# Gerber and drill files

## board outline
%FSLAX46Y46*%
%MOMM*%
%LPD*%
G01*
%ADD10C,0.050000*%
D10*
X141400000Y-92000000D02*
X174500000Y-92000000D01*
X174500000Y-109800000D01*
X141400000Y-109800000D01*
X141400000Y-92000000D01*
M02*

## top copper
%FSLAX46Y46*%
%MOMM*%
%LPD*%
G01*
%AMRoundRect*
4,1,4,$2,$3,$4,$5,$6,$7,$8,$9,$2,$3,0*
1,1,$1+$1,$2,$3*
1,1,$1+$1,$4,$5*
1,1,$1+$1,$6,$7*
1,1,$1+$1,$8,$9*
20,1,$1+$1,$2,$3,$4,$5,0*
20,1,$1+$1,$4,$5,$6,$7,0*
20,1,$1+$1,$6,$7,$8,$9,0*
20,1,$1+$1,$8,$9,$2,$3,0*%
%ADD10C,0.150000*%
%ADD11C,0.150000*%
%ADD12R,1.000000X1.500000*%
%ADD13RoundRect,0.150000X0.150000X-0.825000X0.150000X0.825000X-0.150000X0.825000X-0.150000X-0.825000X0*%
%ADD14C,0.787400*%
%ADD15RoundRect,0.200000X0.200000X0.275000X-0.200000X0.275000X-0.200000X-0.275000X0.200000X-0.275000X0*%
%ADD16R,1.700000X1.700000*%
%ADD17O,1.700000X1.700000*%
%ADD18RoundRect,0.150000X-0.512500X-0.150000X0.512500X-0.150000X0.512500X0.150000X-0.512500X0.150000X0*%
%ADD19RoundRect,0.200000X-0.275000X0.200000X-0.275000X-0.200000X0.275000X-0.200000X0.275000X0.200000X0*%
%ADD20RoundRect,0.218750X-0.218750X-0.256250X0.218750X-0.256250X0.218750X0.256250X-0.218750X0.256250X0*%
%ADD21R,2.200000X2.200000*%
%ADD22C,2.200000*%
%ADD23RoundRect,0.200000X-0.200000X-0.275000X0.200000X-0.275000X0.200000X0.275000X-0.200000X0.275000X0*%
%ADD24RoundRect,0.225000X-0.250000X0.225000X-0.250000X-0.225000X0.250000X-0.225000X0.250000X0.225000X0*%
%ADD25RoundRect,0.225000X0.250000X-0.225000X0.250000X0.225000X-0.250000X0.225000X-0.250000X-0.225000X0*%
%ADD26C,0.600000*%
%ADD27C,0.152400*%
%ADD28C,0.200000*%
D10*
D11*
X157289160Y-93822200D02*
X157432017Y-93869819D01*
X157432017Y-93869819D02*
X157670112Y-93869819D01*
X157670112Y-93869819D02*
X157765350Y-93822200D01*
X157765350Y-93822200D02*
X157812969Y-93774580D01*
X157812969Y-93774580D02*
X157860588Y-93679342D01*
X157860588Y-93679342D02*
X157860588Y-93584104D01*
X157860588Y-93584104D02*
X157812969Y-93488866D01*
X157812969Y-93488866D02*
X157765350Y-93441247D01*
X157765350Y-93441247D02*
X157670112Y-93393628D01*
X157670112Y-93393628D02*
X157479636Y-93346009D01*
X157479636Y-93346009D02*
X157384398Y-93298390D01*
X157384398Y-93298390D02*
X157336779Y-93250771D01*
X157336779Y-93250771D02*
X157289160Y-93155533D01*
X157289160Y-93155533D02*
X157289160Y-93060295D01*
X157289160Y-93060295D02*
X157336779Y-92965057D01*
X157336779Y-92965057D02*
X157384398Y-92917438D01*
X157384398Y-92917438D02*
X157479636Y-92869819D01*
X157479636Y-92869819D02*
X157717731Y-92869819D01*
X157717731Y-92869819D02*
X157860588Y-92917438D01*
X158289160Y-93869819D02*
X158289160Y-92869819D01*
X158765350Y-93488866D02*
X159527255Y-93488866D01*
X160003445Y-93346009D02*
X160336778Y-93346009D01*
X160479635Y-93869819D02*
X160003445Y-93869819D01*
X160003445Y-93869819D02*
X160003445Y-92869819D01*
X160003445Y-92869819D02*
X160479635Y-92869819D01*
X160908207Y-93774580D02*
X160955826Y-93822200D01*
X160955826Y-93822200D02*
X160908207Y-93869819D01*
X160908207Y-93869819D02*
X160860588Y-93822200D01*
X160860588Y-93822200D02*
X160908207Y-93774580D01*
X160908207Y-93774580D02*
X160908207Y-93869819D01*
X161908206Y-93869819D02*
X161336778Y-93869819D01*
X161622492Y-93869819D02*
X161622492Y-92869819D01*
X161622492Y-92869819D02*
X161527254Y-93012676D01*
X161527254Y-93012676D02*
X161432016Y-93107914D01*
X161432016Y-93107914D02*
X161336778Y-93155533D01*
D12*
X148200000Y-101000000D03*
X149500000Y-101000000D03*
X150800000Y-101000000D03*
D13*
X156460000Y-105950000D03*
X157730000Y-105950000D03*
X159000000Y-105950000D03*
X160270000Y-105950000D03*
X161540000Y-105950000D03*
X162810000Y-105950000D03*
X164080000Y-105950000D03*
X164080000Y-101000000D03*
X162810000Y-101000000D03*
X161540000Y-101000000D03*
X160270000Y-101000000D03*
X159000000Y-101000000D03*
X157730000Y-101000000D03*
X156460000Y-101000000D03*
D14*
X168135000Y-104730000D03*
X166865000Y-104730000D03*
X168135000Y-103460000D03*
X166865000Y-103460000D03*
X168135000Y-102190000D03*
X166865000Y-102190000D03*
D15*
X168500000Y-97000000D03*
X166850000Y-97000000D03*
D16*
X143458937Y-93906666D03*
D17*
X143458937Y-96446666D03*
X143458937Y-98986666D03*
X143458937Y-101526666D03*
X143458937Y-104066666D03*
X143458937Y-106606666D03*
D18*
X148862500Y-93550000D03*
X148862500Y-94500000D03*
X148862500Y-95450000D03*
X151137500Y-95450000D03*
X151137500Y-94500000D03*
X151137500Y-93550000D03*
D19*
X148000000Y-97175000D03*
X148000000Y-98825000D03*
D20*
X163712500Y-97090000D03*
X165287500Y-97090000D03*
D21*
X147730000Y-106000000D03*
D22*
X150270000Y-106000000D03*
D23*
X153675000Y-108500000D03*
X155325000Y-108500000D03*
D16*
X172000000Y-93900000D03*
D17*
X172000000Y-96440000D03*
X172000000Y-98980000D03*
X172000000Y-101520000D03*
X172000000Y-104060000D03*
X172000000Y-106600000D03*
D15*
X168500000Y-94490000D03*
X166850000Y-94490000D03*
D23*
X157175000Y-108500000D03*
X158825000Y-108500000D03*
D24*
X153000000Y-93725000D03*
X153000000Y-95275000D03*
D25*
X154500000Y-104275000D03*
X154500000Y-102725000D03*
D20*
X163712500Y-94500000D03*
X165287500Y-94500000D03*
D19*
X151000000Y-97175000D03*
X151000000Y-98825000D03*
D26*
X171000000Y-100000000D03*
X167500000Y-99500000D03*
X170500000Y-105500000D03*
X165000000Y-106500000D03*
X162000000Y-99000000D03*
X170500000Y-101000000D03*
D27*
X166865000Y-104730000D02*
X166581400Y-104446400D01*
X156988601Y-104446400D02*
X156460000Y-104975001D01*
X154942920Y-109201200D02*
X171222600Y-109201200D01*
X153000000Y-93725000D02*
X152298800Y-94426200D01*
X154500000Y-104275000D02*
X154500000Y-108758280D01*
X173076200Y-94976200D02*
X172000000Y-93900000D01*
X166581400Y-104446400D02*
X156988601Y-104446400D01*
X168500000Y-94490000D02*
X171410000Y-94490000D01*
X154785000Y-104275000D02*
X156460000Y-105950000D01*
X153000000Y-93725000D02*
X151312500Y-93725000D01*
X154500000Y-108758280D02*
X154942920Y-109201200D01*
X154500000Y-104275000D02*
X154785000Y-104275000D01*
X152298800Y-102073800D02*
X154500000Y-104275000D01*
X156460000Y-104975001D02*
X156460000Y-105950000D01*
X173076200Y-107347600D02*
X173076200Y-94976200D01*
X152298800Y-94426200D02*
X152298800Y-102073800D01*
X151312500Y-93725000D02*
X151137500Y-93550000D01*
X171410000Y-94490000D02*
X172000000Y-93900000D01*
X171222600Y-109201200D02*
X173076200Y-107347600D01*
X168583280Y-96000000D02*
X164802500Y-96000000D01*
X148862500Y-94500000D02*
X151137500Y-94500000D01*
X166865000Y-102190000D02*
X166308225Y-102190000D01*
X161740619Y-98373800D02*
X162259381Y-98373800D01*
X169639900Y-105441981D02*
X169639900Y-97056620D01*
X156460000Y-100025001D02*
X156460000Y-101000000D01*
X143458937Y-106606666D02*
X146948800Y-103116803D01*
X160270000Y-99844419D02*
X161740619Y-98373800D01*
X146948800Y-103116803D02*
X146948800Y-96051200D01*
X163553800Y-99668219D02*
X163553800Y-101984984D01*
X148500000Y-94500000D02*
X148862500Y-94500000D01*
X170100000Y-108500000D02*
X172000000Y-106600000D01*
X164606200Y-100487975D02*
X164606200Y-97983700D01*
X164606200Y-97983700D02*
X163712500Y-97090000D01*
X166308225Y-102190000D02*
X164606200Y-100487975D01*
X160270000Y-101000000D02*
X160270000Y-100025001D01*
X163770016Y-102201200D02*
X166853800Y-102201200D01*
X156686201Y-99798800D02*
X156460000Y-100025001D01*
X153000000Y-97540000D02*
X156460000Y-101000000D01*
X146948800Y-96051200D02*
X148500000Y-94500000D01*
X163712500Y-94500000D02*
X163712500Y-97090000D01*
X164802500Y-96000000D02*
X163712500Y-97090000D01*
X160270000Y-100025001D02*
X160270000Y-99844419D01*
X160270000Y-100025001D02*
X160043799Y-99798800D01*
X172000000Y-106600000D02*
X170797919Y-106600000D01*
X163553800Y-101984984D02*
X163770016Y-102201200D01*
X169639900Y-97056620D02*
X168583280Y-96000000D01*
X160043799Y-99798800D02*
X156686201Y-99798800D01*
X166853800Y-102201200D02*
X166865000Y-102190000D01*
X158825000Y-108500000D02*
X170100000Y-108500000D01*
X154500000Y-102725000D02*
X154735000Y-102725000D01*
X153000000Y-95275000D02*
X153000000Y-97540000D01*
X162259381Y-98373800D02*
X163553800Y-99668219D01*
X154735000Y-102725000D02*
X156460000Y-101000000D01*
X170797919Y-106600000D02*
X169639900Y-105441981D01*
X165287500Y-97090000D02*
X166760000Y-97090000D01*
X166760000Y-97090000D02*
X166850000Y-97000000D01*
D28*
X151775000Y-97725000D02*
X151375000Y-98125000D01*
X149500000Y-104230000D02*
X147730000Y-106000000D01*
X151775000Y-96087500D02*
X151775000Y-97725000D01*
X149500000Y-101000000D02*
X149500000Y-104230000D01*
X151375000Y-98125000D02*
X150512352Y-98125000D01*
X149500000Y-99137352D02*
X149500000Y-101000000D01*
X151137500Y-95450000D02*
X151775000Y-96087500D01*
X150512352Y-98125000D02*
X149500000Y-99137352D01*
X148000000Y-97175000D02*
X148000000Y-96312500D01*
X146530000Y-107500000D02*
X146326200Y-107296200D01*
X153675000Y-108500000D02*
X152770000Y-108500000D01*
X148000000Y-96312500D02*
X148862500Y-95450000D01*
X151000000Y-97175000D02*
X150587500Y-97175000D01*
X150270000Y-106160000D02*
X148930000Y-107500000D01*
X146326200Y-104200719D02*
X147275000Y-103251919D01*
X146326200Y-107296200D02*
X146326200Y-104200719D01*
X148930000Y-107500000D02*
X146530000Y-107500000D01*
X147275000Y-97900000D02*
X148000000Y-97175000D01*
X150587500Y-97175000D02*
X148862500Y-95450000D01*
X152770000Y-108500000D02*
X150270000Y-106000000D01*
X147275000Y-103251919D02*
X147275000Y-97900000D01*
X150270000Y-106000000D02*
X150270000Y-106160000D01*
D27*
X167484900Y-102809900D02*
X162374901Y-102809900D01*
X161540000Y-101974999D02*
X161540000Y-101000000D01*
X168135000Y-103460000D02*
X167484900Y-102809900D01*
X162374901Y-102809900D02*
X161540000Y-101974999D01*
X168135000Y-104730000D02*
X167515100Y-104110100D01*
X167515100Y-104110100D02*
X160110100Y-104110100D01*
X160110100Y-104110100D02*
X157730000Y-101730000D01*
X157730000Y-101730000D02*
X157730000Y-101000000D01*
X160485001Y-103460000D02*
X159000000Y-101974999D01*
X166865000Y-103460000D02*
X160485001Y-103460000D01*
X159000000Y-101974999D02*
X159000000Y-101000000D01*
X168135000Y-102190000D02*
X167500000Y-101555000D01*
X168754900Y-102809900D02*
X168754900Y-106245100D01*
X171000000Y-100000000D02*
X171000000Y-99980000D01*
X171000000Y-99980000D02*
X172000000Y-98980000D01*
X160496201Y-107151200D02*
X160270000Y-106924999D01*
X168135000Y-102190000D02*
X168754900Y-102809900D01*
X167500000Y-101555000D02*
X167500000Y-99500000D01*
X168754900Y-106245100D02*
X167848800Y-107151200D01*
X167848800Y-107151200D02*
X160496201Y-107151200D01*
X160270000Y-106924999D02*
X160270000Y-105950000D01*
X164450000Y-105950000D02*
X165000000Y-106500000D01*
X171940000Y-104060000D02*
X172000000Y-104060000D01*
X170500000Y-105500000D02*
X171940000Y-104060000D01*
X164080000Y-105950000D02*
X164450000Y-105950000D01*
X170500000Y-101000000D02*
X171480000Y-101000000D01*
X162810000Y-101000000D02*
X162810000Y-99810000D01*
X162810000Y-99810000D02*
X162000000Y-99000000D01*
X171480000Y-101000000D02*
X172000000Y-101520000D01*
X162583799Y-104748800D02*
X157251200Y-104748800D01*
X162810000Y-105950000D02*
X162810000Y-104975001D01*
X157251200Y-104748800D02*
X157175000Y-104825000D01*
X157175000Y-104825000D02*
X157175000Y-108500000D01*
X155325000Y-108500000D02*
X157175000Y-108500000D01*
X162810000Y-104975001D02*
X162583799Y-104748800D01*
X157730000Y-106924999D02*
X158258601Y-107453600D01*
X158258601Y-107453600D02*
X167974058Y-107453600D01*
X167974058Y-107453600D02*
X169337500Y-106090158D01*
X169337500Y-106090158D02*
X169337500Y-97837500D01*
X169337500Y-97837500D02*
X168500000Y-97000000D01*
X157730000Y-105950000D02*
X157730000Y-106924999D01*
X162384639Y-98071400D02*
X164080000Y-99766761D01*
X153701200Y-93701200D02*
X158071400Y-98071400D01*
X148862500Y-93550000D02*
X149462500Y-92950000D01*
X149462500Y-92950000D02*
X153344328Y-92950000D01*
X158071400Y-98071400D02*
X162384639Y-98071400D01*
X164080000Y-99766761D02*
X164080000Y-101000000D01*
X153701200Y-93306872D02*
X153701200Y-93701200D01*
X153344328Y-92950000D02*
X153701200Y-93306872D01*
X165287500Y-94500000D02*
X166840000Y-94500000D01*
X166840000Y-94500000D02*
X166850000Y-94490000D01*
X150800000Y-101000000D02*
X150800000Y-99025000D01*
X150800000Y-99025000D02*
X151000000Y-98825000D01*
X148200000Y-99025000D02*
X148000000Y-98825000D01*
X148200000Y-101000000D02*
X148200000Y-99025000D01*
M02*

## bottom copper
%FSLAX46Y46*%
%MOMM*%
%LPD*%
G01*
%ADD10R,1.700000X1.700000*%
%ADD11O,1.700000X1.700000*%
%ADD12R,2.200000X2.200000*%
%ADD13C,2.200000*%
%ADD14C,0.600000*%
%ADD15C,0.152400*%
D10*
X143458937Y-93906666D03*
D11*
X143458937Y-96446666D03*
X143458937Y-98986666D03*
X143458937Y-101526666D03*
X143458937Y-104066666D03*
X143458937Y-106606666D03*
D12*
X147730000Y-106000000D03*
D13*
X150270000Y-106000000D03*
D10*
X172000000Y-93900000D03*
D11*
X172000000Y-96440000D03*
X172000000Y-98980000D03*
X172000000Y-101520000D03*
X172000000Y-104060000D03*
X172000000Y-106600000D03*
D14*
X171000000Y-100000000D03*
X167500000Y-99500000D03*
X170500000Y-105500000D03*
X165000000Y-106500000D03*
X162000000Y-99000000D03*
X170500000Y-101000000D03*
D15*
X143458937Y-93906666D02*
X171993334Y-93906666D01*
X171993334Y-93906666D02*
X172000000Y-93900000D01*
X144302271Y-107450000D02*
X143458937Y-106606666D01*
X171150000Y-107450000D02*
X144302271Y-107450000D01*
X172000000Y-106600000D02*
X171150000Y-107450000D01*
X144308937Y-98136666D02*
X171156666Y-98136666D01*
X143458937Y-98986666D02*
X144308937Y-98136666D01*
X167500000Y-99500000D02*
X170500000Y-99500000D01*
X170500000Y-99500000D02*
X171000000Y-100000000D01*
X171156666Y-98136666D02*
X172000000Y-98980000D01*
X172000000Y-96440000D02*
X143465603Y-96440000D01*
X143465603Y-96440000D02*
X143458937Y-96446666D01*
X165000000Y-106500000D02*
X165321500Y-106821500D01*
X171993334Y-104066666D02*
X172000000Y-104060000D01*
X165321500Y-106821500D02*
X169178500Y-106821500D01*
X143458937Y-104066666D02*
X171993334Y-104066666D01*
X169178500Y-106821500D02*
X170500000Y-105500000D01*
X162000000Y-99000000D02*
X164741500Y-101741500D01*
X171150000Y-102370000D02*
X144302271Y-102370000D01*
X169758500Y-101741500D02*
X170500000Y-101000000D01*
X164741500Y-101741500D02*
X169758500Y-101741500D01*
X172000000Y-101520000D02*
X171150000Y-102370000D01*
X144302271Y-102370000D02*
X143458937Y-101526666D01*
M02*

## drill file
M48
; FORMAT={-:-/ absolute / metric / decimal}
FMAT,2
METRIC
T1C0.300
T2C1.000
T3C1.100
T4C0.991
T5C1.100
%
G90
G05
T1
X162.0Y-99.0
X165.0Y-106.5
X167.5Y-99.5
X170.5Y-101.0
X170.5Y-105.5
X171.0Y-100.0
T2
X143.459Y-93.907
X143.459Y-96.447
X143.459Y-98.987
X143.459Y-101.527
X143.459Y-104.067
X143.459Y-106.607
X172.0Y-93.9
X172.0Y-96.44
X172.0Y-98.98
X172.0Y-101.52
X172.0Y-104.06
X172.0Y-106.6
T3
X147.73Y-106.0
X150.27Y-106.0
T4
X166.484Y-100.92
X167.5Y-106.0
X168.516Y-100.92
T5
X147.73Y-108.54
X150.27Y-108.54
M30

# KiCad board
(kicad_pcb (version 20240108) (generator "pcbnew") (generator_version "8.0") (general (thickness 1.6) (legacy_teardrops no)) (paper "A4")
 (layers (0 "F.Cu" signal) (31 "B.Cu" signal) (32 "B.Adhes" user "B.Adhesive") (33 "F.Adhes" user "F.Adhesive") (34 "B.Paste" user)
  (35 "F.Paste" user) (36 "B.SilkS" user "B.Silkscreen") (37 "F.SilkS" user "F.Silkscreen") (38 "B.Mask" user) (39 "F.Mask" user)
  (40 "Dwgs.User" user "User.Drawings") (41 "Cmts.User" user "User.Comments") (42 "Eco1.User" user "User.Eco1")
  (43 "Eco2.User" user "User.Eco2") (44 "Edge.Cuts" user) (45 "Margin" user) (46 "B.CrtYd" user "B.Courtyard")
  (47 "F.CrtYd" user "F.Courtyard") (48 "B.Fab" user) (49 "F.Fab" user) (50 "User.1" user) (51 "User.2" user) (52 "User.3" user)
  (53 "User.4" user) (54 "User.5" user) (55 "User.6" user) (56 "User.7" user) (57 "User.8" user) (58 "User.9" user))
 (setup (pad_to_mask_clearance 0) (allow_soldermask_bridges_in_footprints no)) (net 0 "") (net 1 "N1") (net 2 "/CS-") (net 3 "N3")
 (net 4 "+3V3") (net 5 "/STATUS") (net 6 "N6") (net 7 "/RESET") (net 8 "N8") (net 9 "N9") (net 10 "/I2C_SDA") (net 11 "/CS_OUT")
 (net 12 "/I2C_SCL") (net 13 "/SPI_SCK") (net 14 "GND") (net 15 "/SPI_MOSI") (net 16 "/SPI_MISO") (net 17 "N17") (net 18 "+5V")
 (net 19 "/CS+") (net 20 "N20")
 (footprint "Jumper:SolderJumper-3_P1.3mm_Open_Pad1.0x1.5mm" (layer "F.Cu") (at 149.5 101)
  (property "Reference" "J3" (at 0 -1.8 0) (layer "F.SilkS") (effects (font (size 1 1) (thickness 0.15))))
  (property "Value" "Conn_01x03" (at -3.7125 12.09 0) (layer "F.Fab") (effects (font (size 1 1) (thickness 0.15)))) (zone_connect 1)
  (pad "1" smd rect (at -1.3 0) (size 1 1.5) (layers "F.Cu" "F.Mask") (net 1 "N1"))
  (pad "2" smd rect (at 0 0) (size 1 1.5) (layers "F.Cu" "F.Mask") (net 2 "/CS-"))
  (pad "3" smd rect (at 1.3 0) (size 1 1.5) (layers "F.Cu" "F.Mask") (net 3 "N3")))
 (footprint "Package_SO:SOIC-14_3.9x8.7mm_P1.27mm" (layer "F.Cu") (at 160.27 103.475 90)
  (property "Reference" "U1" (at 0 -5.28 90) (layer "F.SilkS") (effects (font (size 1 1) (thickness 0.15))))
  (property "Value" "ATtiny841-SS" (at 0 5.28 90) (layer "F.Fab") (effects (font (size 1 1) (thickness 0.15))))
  (pad "1" smd roundrect (at -2.475 -3.81 90) (size 1.95 0.6) (layers "F.Cu" "F.Paste" "F.Mask") (roundrect_rratio 0.25) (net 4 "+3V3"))
  (pad "2" smd roundrect (at -2.475 -2.54 90) (size 1.95 0.6) (layers "F.Cu" "F.Paste" "F.Mask") (roundrect_rratio 0.25) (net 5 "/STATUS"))
  (pad "3" smd roundrect (at -2.475 -1.27 90) (size 1.95 0.6) (layers "F.Cu" "F.Paste" "F.Mask") (roundrect_rratio 0.25) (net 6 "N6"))
  (pad "4" smd roundrect (at -2.475 0 90) (size 1.95 0.6) (layers "F.Cu" "F.Paste" "F.Mask") (roundrect_rratio 0.25) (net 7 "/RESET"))
  (pad "5" smd roundrect (at -2.475 1.27 90) (size 1.95 0.6) (layers "F.Cu" "F.Paste" "F.Mask") (roundrect_rratio 0.25) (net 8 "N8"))
  (pad "6" smd roundrect (at -2.475 2.54 90) (size 1.95 0.6) (layers "F.Cu" "F.Paste" "F.Mask") (roundrect_rratio 0.25) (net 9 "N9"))
  (pad "7" smd roundrect (at -2.475 3.81 90) (size 1.95 0.6) (layers "F.Cu" "F.Paste" "F.Mask") (roundrect_rratio 0.25) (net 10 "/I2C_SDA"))
  (pad "8" smd roundrect (at 2.475 3.81 90) (size 1.95 0.6) (layers "F.Cu" "F.Paste" "F.Mask") (roundrect_rratio 0.25) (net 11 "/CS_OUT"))
  (pad "9" smd roundrect (at 2.475 2.54 90) (size 1.95 0.6) (layers "F.Cu" "F.Paste" "F.Mask") (roundrect_rratio 0.25) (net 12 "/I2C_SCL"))
  (pad "10" smd roundrect (at 2.475 1.27 90) (size 1.95 0.6) (layers "F.Cu" "F.Paste" "F.Mask") (roundrect_rratio 0.25) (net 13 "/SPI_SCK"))
  (pad "11" smd roundrect (at 2.475 0 90) (size 1.95 0.6) (layers "F.Cu" "F.Paste" "F.Mask") (roundrect_rratio 0.25) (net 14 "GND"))
  (pad "12" smd roundrect (at 2.475 -1.27 90) (size 1.95 0.6) (layers "F.Cu" "F.Paste" "F.Mask") (roundrect_rratio 0.25)
   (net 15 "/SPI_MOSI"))
  (pad "13" smd roundrect (at 2.475 -2.54 90) (size 1.95 0.6) (layers "F.Cu" "F.Paste" "F.Mask") (roundrect_rratio 0.25)
   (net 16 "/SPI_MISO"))
  (pad "14" smd roundrect (at 2.475 -3.81 90) (size 1.95 0.6) (layers "F.Cu" "F.Paste" "F.Mask") (roundrect_rratio 0.25) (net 14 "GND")))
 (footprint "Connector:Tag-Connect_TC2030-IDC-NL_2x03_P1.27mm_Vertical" (layer "F.Cu") (at 167.5 103.46 90)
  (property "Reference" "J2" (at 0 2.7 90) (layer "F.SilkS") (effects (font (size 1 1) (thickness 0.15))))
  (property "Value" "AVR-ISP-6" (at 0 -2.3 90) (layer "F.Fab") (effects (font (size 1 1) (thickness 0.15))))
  (pad "" np_thru_hole circle (at -2.54 0 90) (size 0.9906 0.9906) (drill 0.9906) (layers "*.Cu" "*.Mask"))
  (pad "" np_thru_hole circle (at 2.54 -1.016 90) (size 0.9906 0.9906) (drill 0.9906) (layers "*.Cu" "*.Mask"))
  (pad "" np_thru_hole circle (at 2.54 1.016 90) (size 0.9906 0.9906) (drill 0.9906) (layers "*.Cu" "*.Mask"))
  (pad "1" connect circle (at -1.27 0.635 90) (size 0.7874 0.7874) (layers "F.Cu" "F.Mask") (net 16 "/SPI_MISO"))
  (pad "2" connect circle (at -1.27 -0.635 90) (size 0.7874 0.7874) (layers "F.Cu" "F.Mask") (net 4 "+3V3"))
  (pad "3" connect circle (at 0 0.635 90) (size 0.7874 0.7874) (layers "F.Cu" "F.Mask") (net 13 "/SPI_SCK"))
  (pad "4" connect circle (at 0 -0.635 90) (size 0.7874 0.7874) (layers "F.Cu" "F.Mask") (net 15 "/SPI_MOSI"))
  (pad "5" connect circle (at 1.27 0.635 90) (size 0.7874 0.7874) (layers "F.Cu" "F.Mask") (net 7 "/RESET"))
  (pad "6" connect circle (at 1.27 -0.635 90) (size 0.7874 0.7874) (layers "F.Cu" "F.Mask") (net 14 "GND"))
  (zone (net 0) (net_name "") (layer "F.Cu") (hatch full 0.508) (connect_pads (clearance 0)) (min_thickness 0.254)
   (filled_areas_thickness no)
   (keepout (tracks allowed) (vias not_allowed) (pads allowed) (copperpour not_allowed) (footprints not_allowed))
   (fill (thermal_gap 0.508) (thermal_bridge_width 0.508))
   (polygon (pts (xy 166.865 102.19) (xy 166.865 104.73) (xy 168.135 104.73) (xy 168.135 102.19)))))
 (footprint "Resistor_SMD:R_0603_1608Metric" (layer "F.Cu") (at 167.675 97 180)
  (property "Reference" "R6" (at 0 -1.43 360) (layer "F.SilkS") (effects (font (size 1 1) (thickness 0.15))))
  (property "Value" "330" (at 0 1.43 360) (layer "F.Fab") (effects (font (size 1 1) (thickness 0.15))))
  (pad "1" smd roundrect (at -0.825 0 180) (size 0.8 0.95) (layers "F.Cu" "F.Paste" "F.Mask") (roundrect_rratio 0.25) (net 5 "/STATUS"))
  (pad "2" smd roundrect (at 0.825 0 180) (size 0.8 0.95) (layers "F.Cu" "F.Paste" "F.Mask") (roundrect_rratio 0.25) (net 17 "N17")))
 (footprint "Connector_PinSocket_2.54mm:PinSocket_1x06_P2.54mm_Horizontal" (layer "F.Cu") (at 143.458937 93.906666)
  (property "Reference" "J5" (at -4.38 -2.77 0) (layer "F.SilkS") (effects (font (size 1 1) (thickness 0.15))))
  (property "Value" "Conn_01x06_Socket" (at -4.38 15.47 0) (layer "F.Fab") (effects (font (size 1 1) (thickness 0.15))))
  (pad "1" thru_hole rect (at 0 0) (size 1.7 1.7) (drill 1) (layers "*.Cu" "*.Mask") (remove_unused_layers no) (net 4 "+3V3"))
  (pad "2" thru_hole oval (at 0 2.54) (size 1.7 1.7) (drill 1) (layers "*.Cu" "*.Mask") (remove_unused_layers no) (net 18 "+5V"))
  (pad "3" thru_hole oval (at 0 5.08) (size 1.7 1.7) (drill 1) (layers "*.Cu" "*.Mask") (remove_unused_layers no) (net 7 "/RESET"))
  (pad "4" thru_hole oval (at 0 7.62) (size 1.7 1.7) (drill 1) (layers "*.Cu" "*.Mask") (remove_unused_layers no) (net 12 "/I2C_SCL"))
  (pad "5" thru_hole oval (at 0 10.16) (size 1.7 1.7) (drill 1) (layers "*.Cu" "*.Mask") (remove_unused_layers no) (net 10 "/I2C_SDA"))
  (pad "6" thru_hole oval (at 0 12.7) (size 1.7 1.7) (drill 1) (layers "*.Cu" "*.Mask") (remove_unused_layers no) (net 14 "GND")))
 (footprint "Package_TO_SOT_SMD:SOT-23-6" (layer "F.Cu") (at 150 94.5)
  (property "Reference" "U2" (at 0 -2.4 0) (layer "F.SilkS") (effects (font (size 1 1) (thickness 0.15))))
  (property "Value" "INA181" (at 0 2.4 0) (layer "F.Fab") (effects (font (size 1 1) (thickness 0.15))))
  (pad "1" smd roundrect (at -1.1375 -0.95) (size 1.325 0.6) (layers "F.Cu" "F.Paste" "F.Mask") (roundrect_rratio 0.25) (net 11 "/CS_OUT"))
  (pad "2" smd roundrect (at -1.1375 0) (size 1.325 0.6) (layers "F.Cu" "F.Paste" "F.Mask") (roundrect_rratio 0.25) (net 14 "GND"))
  (pad "3" smd roundrect (at -1.1375 0.95) (size 1.325 0.6) (layers "F.Cu" "F.Paste" "F.Mask") (roundrect_rratio 0.25) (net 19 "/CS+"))
  (pad "4" smd roundrect (at 1.1375 0.95) (size 1.325 0.6) (layers "F.Cu" "F.Paste" "F.Mask") (roundrect_rratio 0.25) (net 2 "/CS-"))
  (pad "5" smd roundrect (at 1.1375 0) (size 1.325 0.6) (layers "F.Cu" "F.Paste" "F.Mask") (roundrect_rratio 0.25) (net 14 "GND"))
  (pad "6" smd roundrect (at 1.1375 -0.95) (size 1.325 0.6) (layers "F.Cu" "F.Paste" "F.Mask") (roundrect_rratio 0.25) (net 4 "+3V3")))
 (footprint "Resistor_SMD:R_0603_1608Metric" (layer "F.Cu") (at 148 98 -90)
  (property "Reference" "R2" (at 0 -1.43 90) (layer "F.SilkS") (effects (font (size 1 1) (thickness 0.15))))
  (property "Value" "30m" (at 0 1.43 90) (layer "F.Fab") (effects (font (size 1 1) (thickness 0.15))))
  (pad "1" smd roundrect (at -0.825 0 270) (size 0.8 0.95) (layers "F.Cu" "F.Paste" "F.Mask") (roundrect_rratio 0.25) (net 19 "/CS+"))
  (pad "2" smd roundrect (at 0.825 0 270) (size 0.8 0.95) (layers "F.Cu" "F.Paste" "F.Mask") (roundrect_rratio 0.25) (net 1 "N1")))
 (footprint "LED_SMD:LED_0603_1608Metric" (layer "F.Cu") (at 164.5 97.09)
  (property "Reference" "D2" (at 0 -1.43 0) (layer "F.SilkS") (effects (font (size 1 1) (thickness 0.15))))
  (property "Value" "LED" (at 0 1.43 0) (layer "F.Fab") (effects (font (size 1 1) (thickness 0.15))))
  (pad "1" smd roundrect (at -0.7875 0) (size 0.875 0.95) (layers "F.Cu" "F.Paste" "F.Mask") (roundrect_rratio 0.25) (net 14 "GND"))
  (pad "2" smd roundrect (at 0.7875 0) (size 0.875 0.95) (layers "F.Cu" "F.Paste" "F.Mask") (roundrect_rratio 0.25) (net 17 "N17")))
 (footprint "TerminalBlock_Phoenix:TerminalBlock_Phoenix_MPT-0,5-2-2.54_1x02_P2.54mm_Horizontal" (layer "F.Cu") (at 147.73 106)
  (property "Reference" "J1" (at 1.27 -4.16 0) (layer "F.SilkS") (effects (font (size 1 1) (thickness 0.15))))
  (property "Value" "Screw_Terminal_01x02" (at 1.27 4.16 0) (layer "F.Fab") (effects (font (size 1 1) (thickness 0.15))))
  (pad "" np_thru_hole circle (at 0 2.54) (size 1.1 1.1) (drill 1.1) (layers "*.Cu" "*.Mask"))
  (pad "" np_thru_hole circle (at 2.54 2.54) (size 1.1 1.1) (drill 1.1) (layers "*.Cu" "*.Mask"))
  (pad "1" thru_hole rect (at 0 0) (size 2.2 2.2) (drill 1.1) (layers "*.Cu" "*.Mask") (remove_unused_layers no) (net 2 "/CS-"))
  (pad "2" thru_hole circle (at 2.54 0) (size 2.2 2.2) (drill 1.1) (layers "*.Cu" "*.Mask") (remove_unused_layers no) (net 19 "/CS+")))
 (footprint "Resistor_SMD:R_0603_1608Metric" (layer "F.Cu") (at 154.5 108.5)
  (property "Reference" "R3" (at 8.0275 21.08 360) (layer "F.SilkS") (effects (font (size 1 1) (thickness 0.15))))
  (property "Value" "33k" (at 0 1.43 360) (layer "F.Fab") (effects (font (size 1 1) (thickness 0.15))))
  (pad "1" smd roundrect (at -0.825 0) (size 0.8 0.95) (layers "F.Cu" "F.Paste" "F.Mask") (roundrect_rratio 0.25) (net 19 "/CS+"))
  (pad "2" smd roundrect (at 0.825 0) (size 0.8 0.95) (layers "F.Cu" "F.Paste" "F.Mask") (roundrect_rratio 0.25) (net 9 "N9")))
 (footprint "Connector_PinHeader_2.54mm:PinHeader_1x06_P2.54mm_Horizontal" (layer "F.Cu") (at 172 93.9)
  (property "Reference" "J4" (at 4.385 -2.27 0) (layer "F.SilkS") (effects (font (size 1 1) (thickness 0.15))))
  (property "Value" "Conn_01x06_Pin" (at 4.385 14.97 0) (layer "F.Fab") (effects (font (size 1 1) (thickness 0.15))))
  (pad "1" thru_hole rect (at 0 0) (size 1.7 1.7) (drill 1) (layers "*.Cu" "*.Mask") (remove_unused_layers no) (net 4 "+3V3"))
  (pad "2" thru_hole oval (at 0 2.54) (size 1.7 1.7) (drill 1) (layers "*.Cu" "*.Mask") (remove_unused_layers no) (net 18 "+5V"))
  (pad "3" thru_hole oval (at 0 5.08) (size 1.7 1.7) (drill 1) (layers "*.Cu" "*.Mask") (remove_unused_layers no) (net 7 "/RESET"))
  (pad "4" thru_hole oval (at 0 7.62) (size 1.7 1.7) (drill 1) (layers "*.Cu" "*.Mask") (remove_unused_layers no) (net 12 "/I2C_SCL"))
  (pad "5" thru_hole oval (at 0 10.16) (size 1.7 1.7) (drill 1) (layers "*.Cu" "*.Mask") (remove_unused_layers no) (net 10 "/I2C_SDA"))
  (pad "6" thru_hole oval (at 0 12.7) (size 1.7 1.7) (drill 1) (layers "*.Cu" "*.Mask") (remove_unused_layers no) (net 14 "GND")))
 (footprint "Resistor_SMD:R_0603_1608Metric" (layer "F.Cu") (at 167.675 94.49 180)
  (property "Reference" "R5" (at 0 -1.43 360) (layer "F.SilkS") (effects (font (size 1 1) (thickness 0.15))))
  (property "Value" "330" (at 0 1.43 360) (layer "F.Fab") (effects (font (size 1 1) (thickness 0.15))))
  (pad "1" smd roundrect (at -0.825 0 180) (size 0.8 0.95) (layers "F.Cu" "F.Paste" "F.Mask") (roundrect_rratio 0.25) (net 4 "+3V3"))
  (pad "2" smd roundrect (at 0.825 0 180) (size 0.8 0.95) (layers "F.Cu" "F.Paste" "F.Mask") (roundrect_rratio 0.25) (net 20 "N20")))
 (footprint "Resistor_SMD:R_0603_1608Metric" (layer "F.Cu") (at 158 108.5)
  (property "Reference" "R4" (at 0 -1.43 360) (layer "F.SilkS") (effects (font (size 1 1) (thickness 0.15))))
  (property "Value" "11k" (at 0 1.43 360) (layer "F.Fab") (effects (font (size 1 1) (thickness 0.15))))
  (pad "1" smd roundrect (at -0.825 0) (size 0.8 0.95) (layers "F.Cu" "F.Paste" "F.Mask") (roundrect_rratio 0.25) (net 9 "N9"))
  (pad "2" smd roundrect (at 0.825 0) (size 0.8 0.95) (layers "F.Cu" "F.Paste" "F.Mask") (roundrect_rratio 0.25) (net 14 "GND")))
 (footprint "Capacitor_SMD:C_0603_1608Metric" (layer "F.Cu") (at 153 94.5 -90)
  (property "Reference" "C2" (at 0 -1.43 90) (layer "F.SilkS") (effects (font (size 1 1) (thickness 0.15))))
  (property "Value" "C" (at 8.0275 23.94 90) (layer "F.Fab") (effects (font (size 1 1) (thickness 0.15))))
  (pad "1" smd roundrect (at -0.775 0 270) (size 0.9 0.95) (layers "F.Cu" "F.Paste" "F.Mask") (roundrect_rratio 0.25) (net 4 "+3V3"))
  (pad "2" smd roundrect (at 0.775 0 270) (size 0.9 0.95) (layers "F.Cu" "F.Paste" "F.Mask") (roundrect_rratio 0.25) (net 14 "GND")))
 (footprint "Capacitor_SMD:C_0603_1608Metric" (layer "F.Cu") (at 154.5 103.5 90)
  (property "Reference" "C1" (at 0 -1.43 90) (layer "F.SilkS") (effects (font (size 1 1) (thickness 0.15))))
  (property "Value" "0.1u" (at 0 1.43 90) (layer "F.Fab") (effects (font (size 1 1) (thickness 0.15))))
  (pad "1" smd roundrect (at -0.775 0 90) (size 0.9 0.95) (layers "F.Cu" "F.Paste" "F.Mask") (roundrect_rratio 0.25) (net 4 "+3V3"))
  (pad "2" smd roundrect (at 0.775 0 90) (size 0.9 0.95) (layers "F.Cu" "F.Paste" "F.Mask") (roundrect_rratio 0.25) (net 14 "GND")))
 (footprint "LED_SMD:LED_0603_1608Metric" (layer "F.Cu") (at 164.5 94.5)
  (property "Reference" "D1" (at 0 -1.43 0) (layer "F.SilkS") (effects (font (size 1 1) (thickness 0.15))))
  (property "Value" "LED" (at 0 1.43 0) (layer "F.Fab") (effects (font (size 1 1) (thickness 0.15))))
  (pad "1" smd roundrect (at -0.7875 0) (size 0.875 0.95) (layers "F.Cu" "F.Paste" "F.Mask") (roundrect_rratio 0.25) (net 14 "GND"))
  (pad "2" smd roundrect (at 0.7875 0) (size 0.875 0.95) (layers "F.Cu" "F.Paste" "F.Mask") (roundrect_rratio 0.25) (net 20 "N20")))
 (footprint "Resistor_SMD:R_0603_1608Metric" (layer "F.Cu") (at 151 98 -90)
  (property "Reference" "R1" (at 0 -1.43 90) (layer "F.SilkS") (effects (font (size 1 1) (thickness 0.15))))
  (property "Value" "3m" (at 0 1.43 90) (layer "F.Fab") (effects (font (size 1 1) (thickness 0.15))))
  (pad "1" smd roundrect (at -0.825 0 270) (size 0.8 0.95) (layers "F.Cu" "F.Paste" "F.Mask") (roundrect_rratio 0.25) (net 19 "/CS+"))
  (pad "2" smd roundrect (at 0.825 0 270) (size 0.8 0.95) (layers "F.Cu" "F.Paste" "F.Mask") (roundrect_rratio 0.25) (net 3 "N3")))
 (gr_rect (start 141.4 92) (end 174.5 109.8) (stroke (width 0.05) (type default)) (fill none) (layer "Edge.Cuts"))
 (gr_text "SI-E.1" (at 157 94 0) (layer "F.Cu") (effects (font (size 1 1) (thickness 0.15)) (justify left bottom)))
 (segment (start 166.865 104.73) (end 166.5814 104.4464) (width 0.1524) (layer "F.Cu") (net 4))
 (segment (start 156.988601 104.4464) (end 156.46 104.975001) (width 0.1524) (layer "F.Cu") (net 4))
 (segment (start 154.94292 109.2012) (end 171.2226 109.2012) (width 0.1524) (layer "F.Cu") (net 4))
 (segment (start 153 93.725) (end 152.2988 94.4262) (width 0.1524) (layer "F.Cu") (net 4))
 (segment (start 154.5 104.275) (end 154.5 108.75828) (width 0.1524) (layer "F.Cu") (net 4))
 (segment (start 173.0762 94.9762) (end 172 93.9) (width 0.1524) (layer "F.Cu") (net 4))
 (segment (start 166.5814 104.4464) (end 156.988601 104.4464) (width 0.1524) (layer "F.Cu") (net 4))
 (segment (start 168.5 94.49) (end 171.41 94.49) (width 0.1524) (layer "F.Cu") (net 4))
 (segment (start 154.785 104.275) (end 156.46 105.95) (width 0.1524) (layer "F.Cu") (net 4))
 (segment (start 153 93.725) (end 151.3125 93.725) (width 0.1524) (layer "F.Cu") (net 4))
 (segment (start 154.5 108.75828) (end 154.94292 109.2012) (width 0.1524) (layer "F.Cu") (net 4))
 (segment (start 154.5 104.275) (end 154.785 104.275) (width 0.1524) (layer "F.Cu") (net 4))
 (segment (start 152.2988 102.0738) (end 154.5 104.275) (width 0.1524) (layer "F.Cu") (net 4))
 (segment (start 156.46 104.975001) (end 156.46 105.95) (width 0.1524) (layer "F.Cu") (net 4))
 (segment (start 173.0762 107.3476) (end 173.0762 94.9762) (width 0.1524) (layer "F.Cu") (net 4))
 (segment (start 152.2988 94.4262) (end 152.2988 102.0738) (width 0.1524) (layer "F.Cu") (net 4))
 (segment (start 151.3125 93.725) (end 151.1375 93.55) (width 0.1524) (layer "F.Cu") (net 4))
 (segment (start 171.41 94.49) (end 172 93.9) (width 0.1524) (layer "F.Cu") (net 4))
 (segment (start 171.2226 109.2012) (end 173.0762 107.3476) (width 0.1524) (layer "F.Cu") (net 4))
 (segment (start 143.458937 93.906666) (end 171.993334 93.906666) (width 0.1524) (layer "B.Cu") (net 4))
 (segment (start 171.993334 93.906666) (end 172 93.9) (width 0.1524) (layer "B.Cu") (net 4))
 (segment (start 168.58328 96) (end 164.8025 96) (width 0.1524) (layer "F.Cu") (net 14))
 (segment (start 148.8625 94.5) (end 151.1375 94.5) (width 0.1524) (layer "F.Cu") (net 14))
 (segment (start 166.865 102.19) (end 166.308225 102.19) (width 0.1524) (layer "F.Cu") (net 14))
 (segment (start 161.740619 98.3738) (end 162.259381 98.3738) (width 0.1524) (layer "F.Cu") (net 14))
 (segment (start 169.6399 105.441981) (end 169.6399 97.05662) (width 0.1524) (layer "F.Cu") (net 14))
 (segment (start 156.46 100.025001) (end 156.46 101) (width 0.1524) (layer "F.Cu") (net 14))
 (segment (start 143.458937 106.606666) (end 146.9488 103.116803) (width 0.1524) (layer "F.Cu") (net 14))
 (segment (start 160.27 99.844419) (end 161.740619 98.3738) (width 0.1524) (layer "F.Cu") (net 14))
 (segment (start 146.9488 103.116803) (end 146.9488 96.0512) (width 0.1524) (layer "F.Cu") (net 14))
 (segment (start 163.5538 99.668219) (end 163.5538 101.984984) (width 0.1524) (layer "F.Cu") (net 14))
 (segment (start 148.5 94.5) (end 148.8625 94.5) (width 0.1524) (layer "F.Cu") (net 14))
 (segment (start 170.1 108.5) (end 172 106.6) (width 0.1524) (layer "F.Cu") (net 14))
 (segment (start 164.6062 100.487975) (end 164.6062 97.9837) (width 0.1524) (layer "F.Cu") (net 14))
 (segment (start 164.6062 97.9837) (end 163.7125 97.09) (width 0.1524) (layer "F.Cu") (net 14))
 (segment (start 166.308225 102.19) (end 164.6062 100.487975) (width 0.1524) (layer "F.Cu") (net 14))
 (segment (start 160.27 101) (end 160.27 100.025001) (width 0.1524) (layer "F.Cu") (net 14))
 (segment (start 163.770016 102.2012) (end 166.8538 102.2012) (width 0.1524) (layer "F.Cu") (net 14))
 (segment (start 156.686201 99.7988) (end 156.46 100.025001) (width 0.1524) (layer "F.Cu") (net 14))
 (segment (start 153 97.54) (end 156.46 101) (width 0.1524) (layer "F.Cu") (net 14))
 (segment (start 146.9488 96.0512) (end 148.5 94.5) (width 0.1524) (layer "F.Cu") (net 14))
 (segment (start 163.7125 94.5) (end 163.7125 97.09) (width 0.1524) (layer "F.Cu") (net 14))
 (segment (start 164.8025 96) (end 163.7125 97.09) (width 0.1524) (layer "F.Cu") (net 14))
 (segment (start 160.27 100.025001) (end 160.27 99.844419) (width 0.1524) (layer "F.Cu") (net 14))
 (segment (start 160.27 100.025001) (end 160.043799 99.7988) (width 0.1524) (layer "F.Cu") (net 14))
 (segment (start 172 106.6) (end 170.797919 106.6) (width 0.1524) (layer "F.Cu") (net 14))
 (segment (start 163.5538 101.984984) (end 163.770016 102.2012) (width 0.1524) (layer "F.Cu") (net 14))
 (segment (start 169.6399 97.05662) (end 168.58328 96) (width 0.1524) (layer "F.Cu") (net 14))
 (segment (start 160.043799 99.7988) (end 156.686201 99.7988) (width 0.1524) (layer "F.Cu") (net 14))
 (segment (start 166.8538 102.2012) (end 166.865 102.19) (width 0.1524) (layer "F.Cu") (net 14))
 (segment (start 158.825 108.5) (end 170.1 108.5) (width 0.1524) (layer "F.Cu") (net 14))
 (segment (start 154.5 102.725) (end 154.735 102.725) (width 0.1524) (layer "F.Cu") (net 14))
 (segment (start 153 95.275) (end 153 97.54) (width 0.1524) (layer "F.Cu") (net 14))
 (segment (start 162.259381 98.3738) (end 163.5538 99.668219) (width 0.1524) (layer "F.Cu") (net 14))
 (segment (start 154.735 102.725) (end 156.46 101) (width 0.1524) (layer "F.Cu") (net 14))
 (segment (start 170.797919 106.6) (end 169.6399 105.441981) (width 0.1524) (layer "F.Cu") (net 14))
 (segment (start 144.302271 107.45) (end 143.458937 106.606666) (width 0.1524) (layer "B.Cu") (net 14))
 (segment (start 171.15 107.45) (end 144.302271 107.45) (width 0.1524) (layer "B.Cu") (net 14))
 (segment (start 172 106.6) (end 171.15 107.45) (width 0.1524) (layer "B.Cu") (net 14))
 (segment (start 165.2875 97.09) (end 166.76 97.09) (width 0.1524) (layer "F.Cu") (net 17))
 (segment (start 166.76 97.09) (end 166.85 97) (width 0.1524) (layer "F.Cu") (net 17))
 (segment (start 151.775 97.725) (end 151.375 98.125) (width 0.2) (layer "F.Cu") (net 2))
 (segment (start 149.5 104.23) (end 147.73 106) (width 0.2) (layer "F.Cu") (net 2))
 (segment (start 151.775 96.0875) (end 151.775 97.725) (width 0.2) (layer "F.Cu") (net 2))
 (segment (start 149.5 101) (end 149.5 104.23) (width 0.2) (layer "F.Cu") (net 2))
 (segment (start 151.375 98.125) (end 150.512352 98.125) (width 0.2) (layer "F.Cu") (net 2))
 (segment (start 149.5 99.137352) (end 149.5 101) (width 0.2) (layer "F.Cu") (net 2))
 (segment (start 151.1375 95.45) (end 151.775 96.0875) (width 0.2) (layer "F.Cu") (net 2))
 (segment (start 150.512352 98.125) (end 149.5 99.137352) (width 0.2) (layer "F.Cu") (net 2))
 (segment (start 148 97.175) (end 148 96.3125) (width 0.2) (layer "F.Cu") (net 19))
 (segment (start 146.53 107.5) (end 146.3262 107.2962) (width 0.2) (layer "F.Cu") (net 19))
 (segment (start 153.675 108.5) (end 152.77 108.5) (width 0.2) (layer "F.Cu") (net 19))
 (segment (start 148 96.3125) (end 148.8625 95.45) (width 0.2) (layer "F.Cu") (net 19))
 (segment (start 151 97.175) (end 150.5875 97.175) (width 0.2) (layer "F.Cu") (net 19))
 (segment (start 150.27 106.16) (end 148.93 107.5) (width 0.2) (layer "F.Cu") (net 19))
 (segment (start 146.3262 104.200719) (end 147.275 103.251919) (width 0.2) (layer "F.Cu") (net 19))
 (segment (start 146.3262 107.2962) (end 146.3262 104.200719) (width 0.2) (layer "F.Cu") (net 19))
 (segment (start 148.93 107.5) (end 146.53 107.5) (width 0.2) (layer "F.Cu") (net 19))
 (segment (start 147.275 97.9) (end 148 97.175) (width 0.2) (layer "F.Cu") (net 19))
 (segment (start 150.5875 97.175) (end 148.8625 95.45) (width 0.2) (layer "F.Cu") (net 19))
 (segment (start 152.77 108.5) (end 150.27 106) (width 0.2) (layer "F.Cu") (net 19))
 (segment (start 147.275 103.251919) (end 147.275 97.9) (width 0.2) (layer "F.Cu") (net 19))
 (segment (start 150.27 106) (end 150.27 106.16) (width 0.2) (layer "F.Cu") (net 19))
 (segment (start 167.4849 102.8099) (end 162.374901 102.8099) (width 0.1524) (layer "F.Cu") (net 13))
 (segment (start 161.54 101.974999) (end 161.54 101) (width 0.1524) (layer "F.Cu") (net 13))
 (segment (start 168.135 103.46) (end 167.4849 102.8099) (width 0.1524) (layer "F.Cu") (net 13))
 (segment (start 162.374901 102.8099) (end 161.54 101.974999) (width 0.1524) (layer "F.Cu") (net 13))
 (segment (start 168.135 104.73) (end 167.5151 104.1101) (width 0.1524) (layer "F.Cu") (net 16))
 (segment (start 167.5151 104.1101) (end 160.1101 104.1101) (width 0.1524) (layer "F.Cu") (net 16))
 (segment (start 160.1101 104.1101) (end 157.73 101.73) (width 0.1524) (layer "F.Cu") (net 16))
 (segment (start 157.73 101.73) (end 157.73 101) (width 0.1524) (layer "F.Cu") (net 16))
 (segment (start 160.485001 103.46) (end 159 101.974999) (width 0.1524) (layer "F.Cu") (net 15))
 (segment (start 166.865 103.46) (end 160.485001 103.46) (width 0.1524) (layer "F.Cu") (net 15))
 (segment (start 159 101.974999) (end 159 101) (width 0.1524) (layer "F.Cu") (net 15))
 (segment (start 168.135 102.19) (end 167.5 101.555) (width 0.1524) (layer "F.Cu") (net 7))
 (segment (start 168.7549 102.8099) (end 168.7549 106.2451) (width 0.1524) (layer "F.Cu") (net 7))
 (segment (start 171 100) (end 171 99.98) (width 0.1524) (layer "F.Cu") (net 7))
 (segment (start 171 99.98) (end 172 98.98) (width 0.1524) (layer "F.Cu") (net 7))
 (segment (start 160.496201 107.1512) (end 160.27 106.924999) (width 0.1524) (layer "F.Cu") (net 7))
 (segment (start 168.135 102.19) (end 168.7549 102.8099) (width 0.1524) (layer "F.Cu") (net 7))
 (segment (start 167.5 101.555) (end 167.5 99.5) (width 0.1524) (layer "F.Cu") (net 7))
 (segment (start 168.7549 106.2451) (end 167.8488 107.1512) (width 0.1524) (layer "F.Cu") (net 7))
 (segment (start 167.8488 107.1512) (end 160.496201 107.1512) (width 0.1524) (layer "F.Cu") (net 7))
 (segment (start 160.27 106.924999) (end 160.27 105.95) (width 0.1524) (layer "F.Cu") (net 7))
 (via (at 171 100) (size 0.6) (drill 0) (layers "F.Cu" "B.Cu") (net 7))
 (via (at 167.5 99.5) (size 0.6) (drill 0) (layers "F.Cu" "B.Cu") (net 7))
 (segment (start 144.308937 98.136666) (end 171.156666 98.136666) (width 0.1524) (layer "B.Cu") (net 7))
 (segment (start 143.458937 98.986666) (end 144.308937 98.136666) (width 0.1524) (layer "B.Cu") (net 7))
 (segment (start 167.5 99.5) (end 170.5 99.5) (width 0.1524) (layer "B.Cu") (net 7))
 (segment (start 170.5 99.5) (end 171 100) (width 0.1524) (layer "B.Cu") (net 7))
 (segment (start 171.156666 98.136666) (end 172 98.98) (width 0.1524) (layer "B.Cu") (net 7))
 (segment (start 172 96.44) (end 143.465603 96.44) (width 0.1524) (layer "B.Cu") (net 18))
 (segment (start 143.465603 96.44) (end 143.458937 96.446666) (width 0.1524) (layer "B.Cu") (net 18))
 (segment (start 164.45 105.95) (end 165 106.5) (width 0.1524) (layer "F.Cu") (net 10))
 (segment (start 171.94 104.06) (end 172 104.06) (width 0.1524) (layer "F.Cu") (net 10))
 (segment (start 170.5 105.5) (end 171.94 104.06) (width 0.1524) (layer "F.Cu") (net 10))
 (segment (start 164.08 105.95) (end 164.45 105.95) (width 0.1524) (layer "F.Cu") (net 10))
 (via (at 170.5 105.5) (size 0.6) (drill 0) (layers "F.Cu" "B.Cu") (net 10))
 (via (at 165 106.5) (size 0.6) (drill 0) (layers "F.Cu" "B.Cu") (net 10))
 (segment (start 165 106.5) (end 165.3215 106.8215) (width 0.1524) (layer "B.Cu") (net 10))
 (segment (start 171.993334 104.066666) (end 172 104.06) (width 0.1524) (layer "B.Cu") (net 10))
 (segment (start 165.3215 106.8215) (end 169.1785 106.8215) (width 0.1524) (layer "B.Cu") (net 10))
 (segment (start 143.458937 104.066666) (end 171.993334 104.066666) (width 0.1524) (layer "B.Cu") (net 10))
 (segment (start 169.1785 106.8215) (end 170.5 105.5) (width 0.1524) (layer "B.Cu") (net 10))
 (segment (start 170.5 101) (end 171.48 101) (width 0.1524) (layer "F.Cu") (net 12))
 (segment (start 162.81 101) (end 162.81 99.81) (width 0.1524) (layer "F.Cu") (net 12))
 (segment (start 162.81 99.81) (end 162 99) (width 0.1524) (layer "F.Cu") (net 12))
 (segment (start 171.48 101) (end 172 101.52) (width 0.1524) (layer "F.Cu") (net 12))
 (via (at 162 99) (size 0.6) (drill 0) (layers "F.Cu" "B.Cu") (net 12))
 (via (at 170.5 101) (size 0.6) (drill 0) (layers "F.Cu" "B.Cu") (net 12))
 (segment (start 162 99) (end 164.7415 101.7415) (width 0.1524) (layer "B.Cu") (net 12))
 (segment (start 171.15 102.37) (end 144.302271 102.37) (width 0.1524) (layer "B.Cu") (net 12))
 (segment (start 169.7585 101.7415) (end 170.5 101) (width 0.1524) (layer "B.Cu") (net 12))
 (segment (start 164.7415 101.7415) (end 169.7585 101.7415) (width 0.1524) (layer "B.Cu") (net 12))
 (segment (start 172 101.52) (end 171.15 102.37) (width 0.1524) (layer "B.Cu") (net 12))
 (segment (start 144.302271 102.37) (end 143.458937 101.526666) (width 0.1524) (layer "B.Cu") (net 12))
 (segment (start 162.583799 104.7488) (end 157.2512 104.7488) (width 0.1524) (layer "F.Cu") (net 9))
 (segment (start 162.81 105.95) (end 162.81 104.975001) (width 0.1524) (layer "F.Cu") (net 9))
 (segment (start 157.2512 104.7488) (end 157.175 104.825) (width 0.1524) (layer "F.Cu") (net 9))
 (segment (start 157.175 104.825) (end 157.175 108.5) (width 0.1524) (layer "F.Cu") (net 9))
 (segment (start 155.325 108.5) (end 157.175 108.5) (width 0.1524) (layer "F.Cu") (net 9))
 (segment (start 162.81 104.975001) (end 162.583799 104.7488) (width 0.1524) (layer "F.Cu") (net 9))
 (segment (start 157.73 106.924999) (end 158.258601 107.4536) (width 0.1524) (layer "F.Cu") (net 5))
 (segment (start 158.258601 107.4536) (end 167.974058 107.4536) (width 0.1524) (layer "F.Cu") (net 5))
 (segment (start 167.974058 107.4536) (end 169.3375 106.090158) (width 0.1524) (layer "F.Cu") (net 5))
 (segment (start 169.3375 106.090158) (end 169.3375 97.8375) (width 0.1524) (layer "F.Cu") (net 5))
 (segment (start 169.3375 97.8375) (end 168.5 97) (width 0.1524) (layer "F.Cu") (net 5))
 (segment (start 157.73 105.95) (end 157.73 106.924999) (width 0.1524) (layer "F.Cu") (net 5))
 (segment (start 162.384639 98.0714) (end 164.08 99.766761) (width 0.1524) (layer "F.Cu") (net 11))
 (segment (start 153.7012 93.7012) (end 158.0714 98.0714) (width 0.1524) (layer "F.Cu") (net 11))
 (segment (start 148.8625 93.55) (end 149.4625 92.95) (width 0.1524) (layer "F.Cu") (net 11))
 (segment (start 149.4625 92.95) (end 153.344328 92.95) (width 0.1524) (layer "F.Cu") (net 11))
 (segment (start 158.0714 98.0714) (end 162.384639 98.0714) (width 0.1524) (layer "F.Cu") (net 11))
 (segment (start 164.08 99.766761) (end 164.08 101) (width 0.1524) (layer "F.Cu") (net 11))
 (segment (start 153.7012 93.306872) (end 153.7012 93.7012) (width 0.1524) (layer "F.Cu") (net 11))
 (segment (start 153.344328 92.95) (end 153.7012 93.306872) (width 0.1524) (layer "F.Cu") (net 11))
 (segment (start 165.2875 94.5) (end 166.84 94.5) (width 0.1524) (layer "F.Cu") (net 20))
 (segment (start 166.84 94.5) (end 166.85 94.49) (width 0.1524) (layer "F.Cu") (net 20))
 (segment (start 150.8 101) (end 150.8 99.025) (width 0.1524) (layer "F.Cu") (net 3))
 (segment (start 150.8 99.025) (end 151 98.825) (width 0.1524) (layer "F.Cu") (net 3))
 (segment (start 148.2 99.025) (end 148 98.825) (width 0.1524) (layer "F.Cu") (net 1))
 (segment (start 148.2 101) (end 148.2 99.025) (width 0.1524) (layer "F.Cu") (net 1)))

